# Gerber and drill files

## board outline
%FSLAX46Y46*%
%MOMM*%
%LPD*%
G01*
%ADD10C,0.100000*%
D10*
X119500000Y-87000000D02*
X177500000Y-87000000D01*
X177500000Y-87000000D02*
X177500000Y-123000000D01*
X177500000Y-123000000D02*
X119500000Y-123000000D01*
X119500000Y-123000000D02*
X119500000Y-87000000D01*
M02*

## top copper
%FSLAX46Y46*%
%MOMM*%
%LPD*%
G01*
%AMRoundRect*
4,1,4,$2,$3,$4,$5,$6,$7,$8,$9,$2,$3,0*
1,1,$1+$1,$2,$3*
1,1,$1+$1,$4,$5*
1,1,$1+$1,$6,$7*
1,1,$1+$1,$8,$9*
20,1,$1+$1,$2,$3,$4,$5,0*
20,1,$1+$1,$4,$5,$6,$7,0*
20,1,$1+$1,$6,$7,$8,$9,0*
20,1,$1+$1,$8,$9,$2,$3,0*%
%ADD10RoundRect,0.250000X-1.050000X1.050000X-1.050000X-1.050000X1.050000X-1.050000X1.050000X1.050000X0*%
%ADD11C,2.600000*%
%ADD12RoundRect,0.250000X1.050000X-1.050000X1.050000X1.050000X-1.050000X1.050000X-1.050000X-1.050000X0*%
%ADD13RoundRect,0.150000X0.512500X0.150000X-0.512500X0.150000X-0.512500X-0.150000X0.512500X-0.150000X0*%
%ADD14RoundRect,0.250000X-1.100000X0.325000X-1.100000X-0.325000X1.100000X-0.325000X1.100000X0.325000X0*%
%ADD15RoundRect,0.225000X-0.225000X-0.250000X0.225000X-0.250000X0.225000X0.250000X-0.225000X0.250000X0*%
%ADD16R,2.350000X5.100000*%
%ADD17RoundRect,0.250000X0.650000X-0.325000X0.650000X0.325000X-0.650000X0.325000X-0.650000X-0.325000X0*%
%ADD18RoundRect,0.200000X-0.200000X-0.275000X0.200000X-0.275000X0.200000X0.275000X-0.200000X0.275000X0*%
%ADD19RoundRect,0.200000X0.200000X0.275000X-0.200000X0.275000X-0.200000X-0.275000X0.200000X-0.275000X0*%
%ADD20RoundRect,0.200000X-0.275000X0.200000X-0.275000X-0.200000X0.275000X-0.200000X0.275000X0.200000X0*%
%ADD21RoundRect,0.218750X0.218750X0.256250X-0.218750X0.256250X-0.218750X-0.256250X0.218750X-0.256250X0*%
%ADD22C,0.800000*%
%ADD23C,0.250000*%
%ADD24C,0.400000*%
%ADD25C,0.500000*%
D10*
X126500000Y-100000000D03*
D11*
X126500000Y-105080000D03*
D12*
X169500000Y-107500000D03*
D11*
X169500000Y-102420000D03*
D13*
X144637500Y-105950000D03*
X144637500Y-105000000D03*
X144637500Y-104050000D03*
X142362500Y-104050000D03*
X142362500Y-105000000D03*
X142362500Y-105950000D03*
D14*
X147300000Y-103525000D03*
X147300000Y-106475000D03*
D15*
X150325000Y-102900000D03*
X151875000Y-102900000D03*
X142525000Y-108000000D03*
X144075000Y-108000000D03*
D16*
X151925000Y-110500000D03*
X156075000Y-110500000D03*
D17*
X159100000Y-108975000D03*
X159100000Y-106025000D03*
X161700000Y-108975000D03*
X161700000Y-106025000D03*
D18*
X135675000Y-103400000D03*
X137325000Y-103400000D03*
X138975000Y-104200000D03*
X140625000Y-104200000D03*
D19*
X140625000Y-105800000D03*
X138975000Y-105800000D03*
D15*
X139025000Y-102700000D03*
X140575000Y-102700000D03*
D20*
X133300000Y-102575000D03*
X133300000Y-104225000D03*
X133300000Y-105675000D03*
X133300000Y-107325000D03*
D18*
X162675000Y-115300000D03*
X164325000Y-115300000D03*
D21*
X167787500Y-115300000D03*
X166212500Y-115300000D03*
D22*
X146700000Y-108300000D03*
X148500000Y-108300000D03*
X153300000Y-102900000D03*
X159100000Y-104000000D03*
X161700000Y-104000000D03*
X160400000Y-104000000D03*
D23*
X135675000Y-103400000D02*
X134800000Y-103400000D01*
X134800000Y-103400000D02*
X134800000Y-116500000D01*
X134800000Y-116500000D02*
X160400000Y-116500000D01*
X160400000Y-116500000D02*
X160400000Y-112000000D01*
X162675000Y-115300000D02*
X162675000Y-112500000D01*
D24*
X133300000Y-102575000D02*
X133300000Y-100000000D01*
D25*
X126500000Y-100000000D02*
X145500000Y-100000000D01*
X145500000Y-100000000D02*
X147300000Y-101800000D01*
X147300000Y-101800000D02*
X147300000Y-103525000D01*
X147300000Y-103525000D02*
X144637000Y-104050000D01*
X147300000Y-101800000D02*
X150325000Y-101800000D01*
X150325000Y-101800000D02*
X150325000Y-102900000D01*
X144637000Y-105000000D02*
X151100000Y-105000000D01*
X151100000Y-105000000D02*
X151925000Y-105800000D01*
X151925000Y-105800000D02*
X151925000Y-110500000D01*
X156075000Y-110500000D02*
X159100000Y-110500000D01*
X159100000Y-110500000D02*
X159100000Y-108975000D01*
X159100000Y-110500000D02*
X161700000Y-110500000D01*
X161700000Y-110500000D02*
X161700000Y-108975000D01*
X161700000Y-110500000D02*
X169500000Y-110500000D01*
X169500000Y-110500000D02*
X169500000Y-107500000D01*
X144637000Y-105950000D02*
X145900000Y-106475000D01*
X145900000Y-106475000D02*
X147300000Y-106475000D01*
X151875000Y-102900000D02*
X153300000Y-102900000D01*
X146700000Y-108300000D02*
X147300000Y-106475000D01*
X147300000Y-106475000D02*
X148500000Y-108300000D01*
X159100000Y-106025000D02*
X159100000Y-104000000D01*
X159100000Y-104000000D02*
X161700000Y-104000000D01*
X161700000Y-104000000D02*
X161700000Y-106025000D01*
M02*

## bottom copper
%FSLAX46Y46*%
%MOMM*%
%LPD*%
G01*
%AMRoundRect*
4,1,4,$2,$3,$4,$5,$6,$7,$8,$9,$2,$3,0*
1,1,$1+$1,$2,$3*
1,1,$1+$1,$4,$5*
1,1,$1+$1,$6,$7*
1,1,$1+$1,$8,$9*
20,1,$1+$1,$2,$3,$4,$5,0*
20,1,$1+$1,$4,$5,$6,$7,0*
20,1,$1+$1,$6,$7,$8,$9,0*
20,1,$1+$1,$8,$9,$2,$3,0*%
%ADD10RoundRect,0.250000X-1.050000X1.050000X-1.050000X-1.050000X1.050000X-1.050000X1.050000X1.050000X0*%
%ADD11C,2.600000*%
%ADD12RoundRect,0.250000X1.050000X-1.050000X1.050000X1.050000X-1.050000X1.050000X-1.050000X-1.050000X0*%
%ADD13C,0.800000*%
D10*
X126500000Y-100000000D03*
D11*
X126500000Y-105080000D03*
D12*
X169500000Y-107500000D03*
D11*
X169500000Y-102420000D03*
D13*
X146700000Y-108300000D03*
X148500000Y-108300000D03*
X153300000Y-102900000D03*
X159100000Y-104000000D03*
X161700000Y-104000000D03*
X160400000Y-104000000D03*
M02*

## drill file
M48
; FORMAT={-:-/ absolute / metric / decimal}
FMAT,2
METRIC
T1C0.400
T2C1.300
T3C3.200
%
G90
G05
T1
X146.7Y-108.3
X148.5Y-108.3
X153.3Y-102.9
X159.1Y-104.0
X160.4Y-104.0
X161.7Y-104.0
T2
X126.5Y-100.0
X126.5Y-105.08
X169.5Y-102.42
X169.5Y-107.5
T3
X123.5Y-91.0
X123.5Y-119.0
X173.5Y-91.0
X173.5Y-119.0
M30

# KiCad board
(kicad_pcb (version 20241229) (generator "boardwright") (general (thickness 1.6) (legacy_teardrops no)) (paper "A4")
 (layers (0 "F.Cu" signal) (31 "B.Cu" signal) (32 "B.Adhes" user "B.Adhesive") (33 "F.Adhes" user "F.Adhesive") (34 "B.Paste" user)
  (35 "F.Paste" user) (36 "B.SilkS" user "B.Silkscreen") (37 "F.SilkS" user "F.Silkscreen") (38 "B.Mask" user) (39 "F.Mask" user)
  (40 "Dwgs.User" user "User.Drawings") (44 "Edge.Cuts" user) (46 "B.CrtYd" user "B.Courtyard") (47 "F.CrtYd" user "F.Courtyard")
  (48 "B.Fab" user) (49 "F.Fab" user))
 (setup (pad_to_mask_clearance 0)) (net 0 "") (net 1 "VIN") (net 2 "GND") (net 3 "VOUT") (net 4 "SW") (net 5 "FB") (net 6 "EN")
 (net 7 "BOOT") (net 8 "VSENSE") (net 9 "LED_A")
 (gr_line (start 119.5 87) (end 177.5 87) (stroke (width 0.1) (type default)) (layer "Edge.Cuts"))
 (gr_line (start 177.5 87) (end 177.5 123) (stroke (width 0.1) (type default)) (layer "Edge.Cuts"))
 (gr_line (start 177.5 123) (end 119.5 123) (stroke (width 0.1) (type default)) (layer "Edge.Cuts"))
 (gr_line (start 119.5 123) (end 119.5 87) (stroke (width 0.1) (type default)) (layer "Edge.Cuts"))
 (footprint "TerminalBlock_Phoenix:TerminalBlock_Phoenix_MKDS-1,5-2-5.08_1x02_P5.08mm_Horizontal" (layer "F.Cu") (at 126.5 100 -90)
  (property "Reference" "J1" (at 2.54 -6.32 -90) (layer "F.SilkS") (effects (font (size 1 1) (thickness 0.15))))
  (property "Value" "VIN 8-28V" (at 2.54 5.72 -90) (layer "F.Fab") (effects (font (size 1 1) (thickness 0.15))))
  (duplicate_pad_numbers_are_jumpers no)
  (pad "1" thru_hole roundrect (at 0 0 -90) (size 2.6 2.6) (drill 1.3) (layers "*.Cu" "*.Mask") (remove_unused_layers no)
   (roundrect_rratio 0.096154) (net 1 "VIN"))
  (pad "2" thru_hole circle (at 5.08 0 -90) (size 2.6 2.6) (drill 1.3) (layers "*.Cu" "*.Mask") (remove_unused_layers no) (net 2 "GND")))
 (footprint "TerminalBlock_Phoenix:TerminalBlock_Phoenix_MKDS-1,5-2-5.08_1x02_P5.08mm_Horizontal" (layer "F.Cu") (at 169.5 107.5 90)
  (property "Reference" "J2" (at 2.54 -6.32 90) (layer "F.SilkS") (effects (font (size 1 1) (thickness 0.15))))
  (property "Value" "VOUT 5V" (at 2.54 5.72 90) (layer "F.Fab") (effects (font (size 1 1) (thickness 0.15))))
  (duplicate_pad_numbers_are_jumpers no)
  (pad "1" thru_hole roundrect (at 0 0 90) (size 2.6 2.6) (drill 1.3) (layers "*.Cu" "*.Mask") (remove_unused_layers no)
   (roundrect_rratio 0.096154) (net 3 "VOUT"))
  (pad "2" thru_hole circle (at 5.08 0 90) (size 2.6 2.6) (drill 1.3) (layers "*.Cu" "*.Mask") (remove_unused_layers no) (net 2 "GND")))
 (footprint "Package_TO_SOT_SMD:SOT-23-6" (layer "F.Cu") (at 143.5 105 180)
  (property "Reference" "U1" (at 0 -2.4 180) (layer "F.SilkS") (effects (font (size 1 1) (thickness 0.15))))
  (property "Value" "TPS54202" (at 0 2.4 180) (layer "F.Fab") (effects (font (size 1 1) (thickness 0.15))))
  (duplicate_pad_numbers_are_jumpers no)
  (pad "1" smd roundrect (at -1.1375 -0.95 180) (size 1.325 0.6) (layers "F.Cu" "F.Mask" "F.Paste") (roundrect_rratio 0.25) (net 2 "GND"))
  (pad "2" smd roundrect (at -1.1375 0 180) (size 1.325 0.6) (layers "F.Cu" "F.Mask" "F.Paste") (roundrect_rratio 0.25) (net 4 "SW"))
  (pad "3" smd roundrect (at -1.1375 0.95 180) (size 1.325 0.6) (layers "F.Cu" "F.Mask" "F.Paste") (roundrect_rratio 0.25) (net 1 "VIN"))
  (pad "4" smd roundrect (at 1.1375 0.95 180) (size 1.325 0.6) (layers "F.Cu" "F.Mask" "F.Paste") (roundrect_rratio 0.25) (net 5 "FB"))
  (pad "5" smd roundrect (at 1.1375 0 180) (size 1.325 0.6) (layers "F.Cu" "F.Mask" "F.Paste") (roundrect_rratio 0.25) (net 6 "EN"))
  (pad "6" smd roundrect (at 1.1375 -0.95 180) (size 1.325 0.6) (layers "F.Cu" "F.Mask" "F.Paste") (roundrect_rratio 0.25) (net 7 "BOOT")))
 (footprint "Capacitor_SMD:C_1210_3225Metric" (layer "F.Cu") (at 147.3 105 -90)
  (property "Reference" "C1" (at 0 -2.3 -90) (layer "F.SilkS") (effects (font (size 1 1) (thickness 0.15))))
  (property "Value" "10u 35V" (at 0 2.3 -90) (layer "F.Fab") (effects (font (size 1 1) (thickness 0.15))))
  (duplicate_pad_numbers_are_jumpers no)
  (pad "1" smd roundrect (at -1.475 0 -90) (size 1.15 2.7) (layers "F.Cu" "F.Mask" "F.Paste") (roundrect_rratio 0.217391) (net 1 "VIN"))
  (pad "2" smd roundrect (at 1.475 0 -90) (size 1.15 2.7) (layers "F.Cu" "F.Mask" "F.Paste") (roundrect_rratio 0.217391) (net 2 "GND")))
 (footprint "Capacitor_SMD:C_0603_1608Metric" (layer "F.Cu") (at 151.1 102.9)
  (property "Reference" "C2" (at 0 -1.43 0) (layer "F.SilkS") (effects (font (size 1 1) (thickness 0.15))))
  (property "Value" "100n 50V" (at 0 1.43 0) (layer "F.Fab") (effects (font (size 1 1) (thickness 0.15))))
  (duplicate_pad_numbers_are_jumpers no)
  (pad "1" smd roundrect (at -0.775 0) (size 0.9 0.95) (layers "F.Cu" "F.Mask" "F.Paste") (roundrect_rratio 0.25) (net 1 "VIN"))
  (pad "2" smd roundrect (at 0.775 0) (size 0.9 0.95) (layers "F.Cu" "F.Mask" "F.Paste") (roundrect_rratio 0.25) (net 2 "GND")))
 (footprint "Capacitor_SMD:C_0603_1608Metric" (layer "F.Cu") (at 143.3 108)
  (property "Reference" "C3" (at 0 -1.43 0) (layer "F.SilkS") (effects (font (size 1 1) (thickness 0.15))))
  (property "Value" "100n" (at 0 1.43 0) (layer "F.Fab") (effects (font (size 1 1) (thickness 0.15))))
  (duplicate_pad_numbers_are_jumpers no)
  (pad "1" smd roundrect (at -0.775 0) (size 0.9 0.95) (layers "F.Cu" "F.Mask" "F.Paste") (roundrect_rratio 0.25) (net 7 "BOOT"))
  (pad "2" smd roundrect (at 0.775 0) (size 0.9 0.95) (layers "F.Cu" "F.Mask" "F.Paste") (roundrect_rratio 0.25) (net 4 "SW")))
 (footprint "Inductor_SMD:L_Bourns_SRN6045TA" (layer "F.Cu") (at 154 110.5)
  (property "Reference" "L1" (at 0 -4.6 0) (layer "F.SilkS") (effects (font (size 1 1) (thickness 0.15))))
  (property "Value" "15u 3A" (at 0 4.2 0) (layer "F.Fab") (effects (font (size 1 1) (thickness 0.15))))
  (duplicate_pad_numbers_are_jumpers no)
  (pad "1" smd rect (at -2.075 0) (size 2.35 5.1) (layers "F.Cu" "F.Mask" "F.Paste") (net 4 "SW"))
  (pad "2" smd rect (at 2.075 0) (size 2.35 5.1) (layers "F.Cu" "F.Mask" "F.Paste") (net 3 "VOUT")))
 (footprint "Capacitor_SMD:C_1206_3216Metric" (layer "F.Cu") (at 159.1 107.5 90)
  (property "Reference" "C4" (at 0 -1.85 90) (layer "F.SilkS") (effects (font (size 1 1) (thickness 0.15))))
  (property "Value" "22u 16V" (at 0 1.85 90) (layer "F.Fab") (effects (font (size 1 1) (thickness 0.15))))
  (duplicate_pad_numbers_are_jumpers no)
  (pad "1" smd roundrect (at -1.475 0 90) (size 1.15 1.8) (layers "F.Cu" "F.Mask" "F.Paste") (roundrect_rratio 0.217391) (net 3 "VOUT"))
  (pad "2" smd roundrect (at 1.475 0 90) (size 1.15 1.8) (layers "F.Cu" "F.Mask" "F.Paste") (roundrect_rratio 0.217391) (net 2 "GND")))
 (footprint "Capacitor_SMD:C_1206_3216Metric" (layer "F.Cu") (at 161.7 107.5 90)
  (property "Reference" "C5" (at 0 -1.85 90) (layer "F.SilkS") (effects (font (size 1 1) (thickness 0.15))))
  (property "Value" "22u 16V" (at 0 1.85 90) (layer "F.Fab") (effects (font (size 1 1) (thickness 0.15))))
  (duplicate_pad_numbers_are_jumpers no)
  (pad "1" smd roundrect (at -1.475 0 90) (size 1.15 1.8) (layers "F.Cu" "F.Mask" "F.Paste") (roundrect_rratio 0.217391) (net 3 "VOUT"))
  (pad "2" smd roundrect (at 1.475 0 90) (size 1.15 1.8) (layers "F.Cu" "F.Mask" "F.Paste") (roundrect_rratio 0.217391) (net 2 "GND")))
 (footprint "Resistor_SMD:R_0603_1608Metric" (layer "F.Cu") (at 136.5 103.4)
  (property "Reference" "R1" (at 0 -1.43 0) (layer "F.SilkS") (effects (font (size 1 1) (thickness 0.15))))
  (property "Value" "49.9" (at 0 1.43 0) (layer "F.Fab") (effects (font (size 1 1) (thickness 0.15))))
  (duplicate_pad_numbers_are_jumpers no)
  (pad "1" smd roundrect (at -0.825 0) (size 0.8 0.95) (layers "F.Cu" "F.Mask" "F.Paste") (roundrect_rratio 0.25) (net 3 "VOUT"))
  (pad "2" smd roundrect (at 0.825 0) (size 0.8 0.95) (layers "F.Cu" "F.Mask" "F.Paste") (roundrect_rratio 0.25) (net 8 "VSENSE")))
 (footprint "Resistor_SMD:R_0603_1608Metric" (layer "F.Cu") (at 139.8 104.2)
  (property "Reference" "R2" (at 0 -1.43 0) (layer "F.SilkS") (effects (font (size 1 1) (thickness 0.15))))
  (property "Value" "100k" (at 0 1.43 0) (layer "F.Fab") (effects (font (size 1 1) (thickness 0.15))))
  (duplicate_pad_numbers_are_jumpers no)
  (pad "1" smd roundrect (at -0.825 0) (size 0.8 0.95) (layers "F.Cu" "F.Mask" "F.Paste") (roundrect_rratio 0.25) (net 8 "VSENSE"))
  (pad "2" smd roundrect (at 0.825 0) (size 0.8 0.95) (layers "F.Cu" "F.Mask" "F.Paste") (roundrect_rratio 0.25) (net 5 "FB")))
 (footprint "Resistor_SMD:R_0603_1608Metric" (layer "F.Cu") (at 139.8 105.8 180)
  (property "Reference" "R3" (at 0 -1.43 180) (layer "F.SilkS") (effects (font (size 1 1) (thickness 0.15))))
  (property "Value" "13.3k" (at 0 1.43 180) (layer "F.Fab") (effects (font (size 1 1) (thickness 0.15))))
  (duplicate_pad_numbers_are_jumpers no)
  (pad "1" smd roundrect (at -0.825 0 180) (size 0.8 0.95) (layers "F.Cu" "F.Mask" "F.Paste") (roundrect_rratio 0.25) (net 5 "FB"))
  (pad "2" smd roundrect (at 0.825 0 180) (size 0.8 0.95) (layers "F.Cu" "F.Mask" "F.Paste") (roundrect_rratio 0.25) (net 2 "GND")))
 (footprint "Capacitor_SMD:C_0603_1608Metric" (layer "F.Cu") (at 139.8 102.7)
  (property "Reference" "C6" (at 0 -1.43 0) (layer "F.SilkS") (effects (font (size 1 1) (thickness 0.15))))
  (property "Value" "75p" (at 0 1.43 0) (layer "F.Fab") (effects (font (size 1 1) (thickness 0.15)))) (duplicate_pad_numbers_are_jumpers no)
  (pad "1" smd roundrect (at -0.775 0) (size 0.9 0.95) (layers "F.Cu" "F.Mask" "F.Paste") (roundrect_rratio 0.25) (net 8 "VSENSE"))
  (pad "2" smd roundrect (at 0.775 0) (size 0.9 0.95) (layers "F.Cu" "F.Mask" "F.Paste") (roundrect_rratio 0.25) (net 5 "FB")))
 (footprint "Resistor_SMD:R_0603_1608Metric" (layer "F.Cu") (at 133.3 103.4 -90)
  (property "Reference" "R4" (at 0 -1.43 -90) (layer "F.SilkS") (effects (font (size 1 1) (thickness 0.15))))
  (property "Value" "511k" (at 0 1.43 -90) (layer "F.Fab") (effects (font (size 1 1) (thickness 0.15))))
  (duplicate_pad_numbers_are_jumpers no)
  (pad "1" smd roundrect (at -0.825 0 -90) (size 0.8 0.95) (layers "F.Cu" "F.Mask" "F.Paste") (roundrect_rratio 0.25) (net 1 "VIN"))
  (pad "2" smd roundrect (at 0.825 0 -90) (size 0.8 0.95) (layers "F.Cu" "F.Mask" "F.Paste") (roundrect_rratio 0.25) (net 6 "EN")))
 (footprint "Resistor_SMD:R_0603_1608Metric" (layer "F.Cu") (at 133.3 106.5 -90)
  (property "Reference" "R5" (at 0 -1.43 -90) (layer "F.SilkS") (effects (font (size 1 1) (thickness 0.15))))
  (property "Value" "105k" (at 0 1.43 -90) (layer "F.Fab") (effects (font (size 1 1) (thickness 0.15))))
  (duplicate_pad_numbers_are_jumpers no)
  (pad "1" smd roundrect (at -0.825 0 -90) (size 0.8 0.95) (layers "F.Cu" "F.Mask" "F.Paste") (roundrect_rratio 0.25) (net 6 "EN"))
  (pad "2" smd roundrect (at 0.825 0 -90) (size 0.8 0.95) (layers "F.Cu" "F.Mask" "F.Paste") (roundrect_rratio 0.25) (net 2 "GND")))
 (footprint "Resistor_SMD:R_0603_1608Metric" (layer "F.Cu") (at 163.5 115.3)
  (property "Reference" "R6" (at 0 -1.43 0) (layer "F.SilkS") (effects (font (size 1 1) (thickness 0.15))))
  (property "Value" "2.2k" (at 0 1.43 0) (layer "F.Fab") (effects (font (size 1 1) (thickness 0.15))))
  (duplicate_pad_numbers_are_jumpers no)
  (pad "1" smd roundrect (at -0.825 0) (size 0.8 0.95) (layers "F.Cu" "F.Mask" "F.Paste") (roundrect_rratio 0.25) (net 3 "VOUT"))
  (pad "2" smd roundrect (at 0.825 0) (size 0.8 0.95) (layers "F.Cu" "F.Mask" "F.Paste") (roundrect_rratio 0.25) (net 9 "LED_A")))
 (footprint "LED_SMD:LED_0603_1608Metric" (layer "F.Cu") (at 167 115.3 180)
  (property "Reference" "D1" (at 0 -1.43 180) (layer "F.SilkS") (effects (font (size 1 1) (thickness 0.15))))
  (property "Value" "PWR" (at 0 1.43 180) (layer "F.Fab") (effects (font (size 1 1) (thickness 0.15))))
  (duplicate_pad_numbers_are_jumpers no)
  (pad "1" smd roundrect (at -0.7875 0 180) (size 0.875 0.95) (layers "F.Cu" "F.Mask" "F.Paste") (roundrect_rratio 0.25) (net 2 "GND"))
  (pad "2" smd roundrect (at 0.7875 0 180) (size 0.875 0.95) (layers "F.Cu" "F.Mask" "F.Paste") (roundrect_rratio 0.25) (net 9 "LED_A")))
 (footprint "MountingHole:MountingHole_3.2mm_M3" (layer "F.Cu") (at 123.5 91)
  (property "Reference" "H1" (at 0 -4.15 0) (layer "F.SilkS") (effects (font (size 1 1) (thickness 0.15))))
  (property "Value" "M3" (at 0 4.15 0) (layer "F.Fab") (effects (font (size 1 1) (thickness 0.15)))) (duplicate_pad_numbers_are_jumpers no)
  (pad "" np_thru_hole circle (at 0 0) (size 3.2 3.2) (drill 3.2) (layers "*.Cu" "*.Mask")))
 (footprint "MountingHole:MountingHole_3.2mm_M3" (layer "F.Cu") (at 173.5 91)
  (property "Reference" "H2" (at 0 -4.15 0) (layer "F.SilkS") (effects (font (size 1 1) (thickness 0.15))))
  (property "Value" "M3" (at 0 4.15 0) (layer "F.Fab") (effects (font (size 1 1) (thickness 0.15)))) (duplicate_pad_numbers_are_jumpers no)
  (pad "" np_thru_hole circle (at 0 0) (size 3.2 3.2) (drill 3.2) (layers "*.Cu" "*.Mask")))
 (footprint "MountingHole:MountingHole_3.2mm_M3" (layer "F.Cu") (at 123.5 119)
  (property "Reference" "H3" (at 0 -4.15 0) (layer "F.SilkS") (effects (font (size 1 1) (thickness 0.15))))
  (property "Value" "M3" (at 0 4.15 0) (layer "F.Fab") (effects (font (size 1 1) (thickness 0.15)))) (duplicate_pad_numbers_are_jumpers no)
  (pad "" np_thru_hole circle (at 0 0) (size 3.2 3.2) (drill 3.2) (layers "*.Cu" "*.Mask")))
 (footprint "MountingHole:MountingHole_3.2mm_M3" (layer "F.Cu") (at 173.5 119)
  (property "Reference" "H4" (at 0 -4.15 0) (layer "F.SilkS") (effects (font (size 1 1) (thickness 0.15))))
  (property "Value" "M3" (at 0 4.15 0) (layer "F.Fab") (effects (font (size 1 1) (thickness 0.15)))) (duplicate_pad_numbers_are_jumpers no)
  (pad "" np_thru_hole circle (at 0 0) (size 3.2 3.2) (drill 3.2) (layers "*.Cu" "*.Mask")))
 (via (at 146.7 108.3) (size 0.8) (drill 0.4) (layers "F.Cu" "B.Cu") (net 2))
 (via (at 148.5 108.3) (size 0.8) (drill 0.4) (layers "F.Cu" "B.Cu") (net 2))
 (via (at 153.3 102.9) (size 0.8) (drill 0.4) (layers "F.Cu" "B.Cu") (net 2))
 (via (at 159.1 104.0) (size 0.8) (drill 0.4) (layers "F.Cu" "B.Cu") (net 2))
 (via (at 161.7 104.0) (size 0.8) (drill 0.4) (layers "F.Cu" "B.Cu") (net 2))
 (via (at 160.4 104.0) (size 0.8) (drill 0.4) (layers "F.Cu" "B.Cu") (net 2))
 (segment (start 135.675 103.4) (end 134.8 103.4) (width 0.25) (layer "F.Cu") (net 3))
 (segment (start 134.8 103.4) (end 134.8 116.5) (width 0.25) (layer "F.Cu") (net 3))
 (segment (start 134.8 116.5) (end 160.4 116.5) (width 0.25) (layer "F.Cu") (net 3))
 (segment (start 160.4 116.5) (end 160.4 112.0) (width 0.25) (layer "F.Cu") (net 3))
 (segment (start 162.675 115.3) (end 162.675 112.5) (width 0.25) (layer "F.Cu") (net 3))
 (segment (start 133.3 102.575) (end 133.3 100.0) (width 0.4) (layer "F.Cu") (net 1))
 (segment (start 126.5 100.0) (end 145.5 100.0) (width 0.5) (layer "F.Cu") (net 1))
 (segment (start 145.5 100.0) (end 147.3 101.8) (width 0.5) (layer "F.Cu") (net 1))
 (segment (start 147.3 101.8) (end 147.3 103.525) (width 0.5) (layer "F.Cu") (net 1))
 (segment (start 147.3 103.525) (end 144.637 104.05) (width 0.5) (layer "F.Cu") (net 1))
 (segment (start 147.3 101.8) (end 150.325 101.8) (width 0.5) (layer "F.Cu") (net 1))
 (segment (start 150.325 101.8) (end 150.325 102.9) (width 0.5) (layer "F.Cu") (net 1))
 (segment (start 144.637 105.0) (end 151.1 105.0) (width 0.5) (layer "F.Cu") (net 4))
 (segment (start 151.1 105.0) (end 151.925 105.8) (width 0.5) (layer "F.Cu") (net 4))
 (segment (start 151.925 105.8) (end 151.925 110.5) (width 0.5) (layer "F.Cu") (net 4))
 (segment (start 156.075 110.5) (end 159.1 110.5) (width 0.5) (layer "F.Cu") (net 3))
 (segment (start 159.1 110.5) (end 159.1 108.975) (width 0.5) (layer "F.Cu") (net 3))
 (segment (start 159.1 110.5) (end 161.7 110.5) (width 0.5) (layer "F.Cu") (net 3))
 (segment (start 161.7 110.5) (end 161.7 108.975) (width 0.5) (layer "F.Cu") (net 3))
 (segment (start 161.7 110.5) (end 169.5 110.5) (width 0.5) (layer "F.Cu") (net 3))
 (segment (start 169.5 110.5) (end 169.5 107.5) (width 0.5) (layer "F.Cu") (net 3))
 (segment (start 144.637 105.95) (end 145.9 106.475) (width 0.5) (layer "F.Cu") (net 2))
 (segment (start 145.9 106.475) (end 147.3 106.475) (width 0.5) (layer "F.Cu") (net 2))
 (segment (start 151.875 102.9) (end 153.3 102.9) (width 0.5) (layer "F.Cu") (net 2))
 (segment (start 146.7 108.3) (end 147.3 106.475) (width 0.5) (layer "F.Cu") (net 2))
 (segment (start 147.3 106.475) (end 148.5 108.3) (width 0.5) (layer "F.Cu") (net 2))
 (segment (start 159.1 106.025) (end 159.1 104.0) (width 0.5) (layer "F.Cu") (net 2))
 (segment (start 159.1 104.0) (end 161.7 104.0) (width 0.5) (layer "F.Cu") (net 2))
 (segment (start 161.7 104.0) (end 161.7 106.025) (width 0.5) (layer "F.Cu") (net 2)))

